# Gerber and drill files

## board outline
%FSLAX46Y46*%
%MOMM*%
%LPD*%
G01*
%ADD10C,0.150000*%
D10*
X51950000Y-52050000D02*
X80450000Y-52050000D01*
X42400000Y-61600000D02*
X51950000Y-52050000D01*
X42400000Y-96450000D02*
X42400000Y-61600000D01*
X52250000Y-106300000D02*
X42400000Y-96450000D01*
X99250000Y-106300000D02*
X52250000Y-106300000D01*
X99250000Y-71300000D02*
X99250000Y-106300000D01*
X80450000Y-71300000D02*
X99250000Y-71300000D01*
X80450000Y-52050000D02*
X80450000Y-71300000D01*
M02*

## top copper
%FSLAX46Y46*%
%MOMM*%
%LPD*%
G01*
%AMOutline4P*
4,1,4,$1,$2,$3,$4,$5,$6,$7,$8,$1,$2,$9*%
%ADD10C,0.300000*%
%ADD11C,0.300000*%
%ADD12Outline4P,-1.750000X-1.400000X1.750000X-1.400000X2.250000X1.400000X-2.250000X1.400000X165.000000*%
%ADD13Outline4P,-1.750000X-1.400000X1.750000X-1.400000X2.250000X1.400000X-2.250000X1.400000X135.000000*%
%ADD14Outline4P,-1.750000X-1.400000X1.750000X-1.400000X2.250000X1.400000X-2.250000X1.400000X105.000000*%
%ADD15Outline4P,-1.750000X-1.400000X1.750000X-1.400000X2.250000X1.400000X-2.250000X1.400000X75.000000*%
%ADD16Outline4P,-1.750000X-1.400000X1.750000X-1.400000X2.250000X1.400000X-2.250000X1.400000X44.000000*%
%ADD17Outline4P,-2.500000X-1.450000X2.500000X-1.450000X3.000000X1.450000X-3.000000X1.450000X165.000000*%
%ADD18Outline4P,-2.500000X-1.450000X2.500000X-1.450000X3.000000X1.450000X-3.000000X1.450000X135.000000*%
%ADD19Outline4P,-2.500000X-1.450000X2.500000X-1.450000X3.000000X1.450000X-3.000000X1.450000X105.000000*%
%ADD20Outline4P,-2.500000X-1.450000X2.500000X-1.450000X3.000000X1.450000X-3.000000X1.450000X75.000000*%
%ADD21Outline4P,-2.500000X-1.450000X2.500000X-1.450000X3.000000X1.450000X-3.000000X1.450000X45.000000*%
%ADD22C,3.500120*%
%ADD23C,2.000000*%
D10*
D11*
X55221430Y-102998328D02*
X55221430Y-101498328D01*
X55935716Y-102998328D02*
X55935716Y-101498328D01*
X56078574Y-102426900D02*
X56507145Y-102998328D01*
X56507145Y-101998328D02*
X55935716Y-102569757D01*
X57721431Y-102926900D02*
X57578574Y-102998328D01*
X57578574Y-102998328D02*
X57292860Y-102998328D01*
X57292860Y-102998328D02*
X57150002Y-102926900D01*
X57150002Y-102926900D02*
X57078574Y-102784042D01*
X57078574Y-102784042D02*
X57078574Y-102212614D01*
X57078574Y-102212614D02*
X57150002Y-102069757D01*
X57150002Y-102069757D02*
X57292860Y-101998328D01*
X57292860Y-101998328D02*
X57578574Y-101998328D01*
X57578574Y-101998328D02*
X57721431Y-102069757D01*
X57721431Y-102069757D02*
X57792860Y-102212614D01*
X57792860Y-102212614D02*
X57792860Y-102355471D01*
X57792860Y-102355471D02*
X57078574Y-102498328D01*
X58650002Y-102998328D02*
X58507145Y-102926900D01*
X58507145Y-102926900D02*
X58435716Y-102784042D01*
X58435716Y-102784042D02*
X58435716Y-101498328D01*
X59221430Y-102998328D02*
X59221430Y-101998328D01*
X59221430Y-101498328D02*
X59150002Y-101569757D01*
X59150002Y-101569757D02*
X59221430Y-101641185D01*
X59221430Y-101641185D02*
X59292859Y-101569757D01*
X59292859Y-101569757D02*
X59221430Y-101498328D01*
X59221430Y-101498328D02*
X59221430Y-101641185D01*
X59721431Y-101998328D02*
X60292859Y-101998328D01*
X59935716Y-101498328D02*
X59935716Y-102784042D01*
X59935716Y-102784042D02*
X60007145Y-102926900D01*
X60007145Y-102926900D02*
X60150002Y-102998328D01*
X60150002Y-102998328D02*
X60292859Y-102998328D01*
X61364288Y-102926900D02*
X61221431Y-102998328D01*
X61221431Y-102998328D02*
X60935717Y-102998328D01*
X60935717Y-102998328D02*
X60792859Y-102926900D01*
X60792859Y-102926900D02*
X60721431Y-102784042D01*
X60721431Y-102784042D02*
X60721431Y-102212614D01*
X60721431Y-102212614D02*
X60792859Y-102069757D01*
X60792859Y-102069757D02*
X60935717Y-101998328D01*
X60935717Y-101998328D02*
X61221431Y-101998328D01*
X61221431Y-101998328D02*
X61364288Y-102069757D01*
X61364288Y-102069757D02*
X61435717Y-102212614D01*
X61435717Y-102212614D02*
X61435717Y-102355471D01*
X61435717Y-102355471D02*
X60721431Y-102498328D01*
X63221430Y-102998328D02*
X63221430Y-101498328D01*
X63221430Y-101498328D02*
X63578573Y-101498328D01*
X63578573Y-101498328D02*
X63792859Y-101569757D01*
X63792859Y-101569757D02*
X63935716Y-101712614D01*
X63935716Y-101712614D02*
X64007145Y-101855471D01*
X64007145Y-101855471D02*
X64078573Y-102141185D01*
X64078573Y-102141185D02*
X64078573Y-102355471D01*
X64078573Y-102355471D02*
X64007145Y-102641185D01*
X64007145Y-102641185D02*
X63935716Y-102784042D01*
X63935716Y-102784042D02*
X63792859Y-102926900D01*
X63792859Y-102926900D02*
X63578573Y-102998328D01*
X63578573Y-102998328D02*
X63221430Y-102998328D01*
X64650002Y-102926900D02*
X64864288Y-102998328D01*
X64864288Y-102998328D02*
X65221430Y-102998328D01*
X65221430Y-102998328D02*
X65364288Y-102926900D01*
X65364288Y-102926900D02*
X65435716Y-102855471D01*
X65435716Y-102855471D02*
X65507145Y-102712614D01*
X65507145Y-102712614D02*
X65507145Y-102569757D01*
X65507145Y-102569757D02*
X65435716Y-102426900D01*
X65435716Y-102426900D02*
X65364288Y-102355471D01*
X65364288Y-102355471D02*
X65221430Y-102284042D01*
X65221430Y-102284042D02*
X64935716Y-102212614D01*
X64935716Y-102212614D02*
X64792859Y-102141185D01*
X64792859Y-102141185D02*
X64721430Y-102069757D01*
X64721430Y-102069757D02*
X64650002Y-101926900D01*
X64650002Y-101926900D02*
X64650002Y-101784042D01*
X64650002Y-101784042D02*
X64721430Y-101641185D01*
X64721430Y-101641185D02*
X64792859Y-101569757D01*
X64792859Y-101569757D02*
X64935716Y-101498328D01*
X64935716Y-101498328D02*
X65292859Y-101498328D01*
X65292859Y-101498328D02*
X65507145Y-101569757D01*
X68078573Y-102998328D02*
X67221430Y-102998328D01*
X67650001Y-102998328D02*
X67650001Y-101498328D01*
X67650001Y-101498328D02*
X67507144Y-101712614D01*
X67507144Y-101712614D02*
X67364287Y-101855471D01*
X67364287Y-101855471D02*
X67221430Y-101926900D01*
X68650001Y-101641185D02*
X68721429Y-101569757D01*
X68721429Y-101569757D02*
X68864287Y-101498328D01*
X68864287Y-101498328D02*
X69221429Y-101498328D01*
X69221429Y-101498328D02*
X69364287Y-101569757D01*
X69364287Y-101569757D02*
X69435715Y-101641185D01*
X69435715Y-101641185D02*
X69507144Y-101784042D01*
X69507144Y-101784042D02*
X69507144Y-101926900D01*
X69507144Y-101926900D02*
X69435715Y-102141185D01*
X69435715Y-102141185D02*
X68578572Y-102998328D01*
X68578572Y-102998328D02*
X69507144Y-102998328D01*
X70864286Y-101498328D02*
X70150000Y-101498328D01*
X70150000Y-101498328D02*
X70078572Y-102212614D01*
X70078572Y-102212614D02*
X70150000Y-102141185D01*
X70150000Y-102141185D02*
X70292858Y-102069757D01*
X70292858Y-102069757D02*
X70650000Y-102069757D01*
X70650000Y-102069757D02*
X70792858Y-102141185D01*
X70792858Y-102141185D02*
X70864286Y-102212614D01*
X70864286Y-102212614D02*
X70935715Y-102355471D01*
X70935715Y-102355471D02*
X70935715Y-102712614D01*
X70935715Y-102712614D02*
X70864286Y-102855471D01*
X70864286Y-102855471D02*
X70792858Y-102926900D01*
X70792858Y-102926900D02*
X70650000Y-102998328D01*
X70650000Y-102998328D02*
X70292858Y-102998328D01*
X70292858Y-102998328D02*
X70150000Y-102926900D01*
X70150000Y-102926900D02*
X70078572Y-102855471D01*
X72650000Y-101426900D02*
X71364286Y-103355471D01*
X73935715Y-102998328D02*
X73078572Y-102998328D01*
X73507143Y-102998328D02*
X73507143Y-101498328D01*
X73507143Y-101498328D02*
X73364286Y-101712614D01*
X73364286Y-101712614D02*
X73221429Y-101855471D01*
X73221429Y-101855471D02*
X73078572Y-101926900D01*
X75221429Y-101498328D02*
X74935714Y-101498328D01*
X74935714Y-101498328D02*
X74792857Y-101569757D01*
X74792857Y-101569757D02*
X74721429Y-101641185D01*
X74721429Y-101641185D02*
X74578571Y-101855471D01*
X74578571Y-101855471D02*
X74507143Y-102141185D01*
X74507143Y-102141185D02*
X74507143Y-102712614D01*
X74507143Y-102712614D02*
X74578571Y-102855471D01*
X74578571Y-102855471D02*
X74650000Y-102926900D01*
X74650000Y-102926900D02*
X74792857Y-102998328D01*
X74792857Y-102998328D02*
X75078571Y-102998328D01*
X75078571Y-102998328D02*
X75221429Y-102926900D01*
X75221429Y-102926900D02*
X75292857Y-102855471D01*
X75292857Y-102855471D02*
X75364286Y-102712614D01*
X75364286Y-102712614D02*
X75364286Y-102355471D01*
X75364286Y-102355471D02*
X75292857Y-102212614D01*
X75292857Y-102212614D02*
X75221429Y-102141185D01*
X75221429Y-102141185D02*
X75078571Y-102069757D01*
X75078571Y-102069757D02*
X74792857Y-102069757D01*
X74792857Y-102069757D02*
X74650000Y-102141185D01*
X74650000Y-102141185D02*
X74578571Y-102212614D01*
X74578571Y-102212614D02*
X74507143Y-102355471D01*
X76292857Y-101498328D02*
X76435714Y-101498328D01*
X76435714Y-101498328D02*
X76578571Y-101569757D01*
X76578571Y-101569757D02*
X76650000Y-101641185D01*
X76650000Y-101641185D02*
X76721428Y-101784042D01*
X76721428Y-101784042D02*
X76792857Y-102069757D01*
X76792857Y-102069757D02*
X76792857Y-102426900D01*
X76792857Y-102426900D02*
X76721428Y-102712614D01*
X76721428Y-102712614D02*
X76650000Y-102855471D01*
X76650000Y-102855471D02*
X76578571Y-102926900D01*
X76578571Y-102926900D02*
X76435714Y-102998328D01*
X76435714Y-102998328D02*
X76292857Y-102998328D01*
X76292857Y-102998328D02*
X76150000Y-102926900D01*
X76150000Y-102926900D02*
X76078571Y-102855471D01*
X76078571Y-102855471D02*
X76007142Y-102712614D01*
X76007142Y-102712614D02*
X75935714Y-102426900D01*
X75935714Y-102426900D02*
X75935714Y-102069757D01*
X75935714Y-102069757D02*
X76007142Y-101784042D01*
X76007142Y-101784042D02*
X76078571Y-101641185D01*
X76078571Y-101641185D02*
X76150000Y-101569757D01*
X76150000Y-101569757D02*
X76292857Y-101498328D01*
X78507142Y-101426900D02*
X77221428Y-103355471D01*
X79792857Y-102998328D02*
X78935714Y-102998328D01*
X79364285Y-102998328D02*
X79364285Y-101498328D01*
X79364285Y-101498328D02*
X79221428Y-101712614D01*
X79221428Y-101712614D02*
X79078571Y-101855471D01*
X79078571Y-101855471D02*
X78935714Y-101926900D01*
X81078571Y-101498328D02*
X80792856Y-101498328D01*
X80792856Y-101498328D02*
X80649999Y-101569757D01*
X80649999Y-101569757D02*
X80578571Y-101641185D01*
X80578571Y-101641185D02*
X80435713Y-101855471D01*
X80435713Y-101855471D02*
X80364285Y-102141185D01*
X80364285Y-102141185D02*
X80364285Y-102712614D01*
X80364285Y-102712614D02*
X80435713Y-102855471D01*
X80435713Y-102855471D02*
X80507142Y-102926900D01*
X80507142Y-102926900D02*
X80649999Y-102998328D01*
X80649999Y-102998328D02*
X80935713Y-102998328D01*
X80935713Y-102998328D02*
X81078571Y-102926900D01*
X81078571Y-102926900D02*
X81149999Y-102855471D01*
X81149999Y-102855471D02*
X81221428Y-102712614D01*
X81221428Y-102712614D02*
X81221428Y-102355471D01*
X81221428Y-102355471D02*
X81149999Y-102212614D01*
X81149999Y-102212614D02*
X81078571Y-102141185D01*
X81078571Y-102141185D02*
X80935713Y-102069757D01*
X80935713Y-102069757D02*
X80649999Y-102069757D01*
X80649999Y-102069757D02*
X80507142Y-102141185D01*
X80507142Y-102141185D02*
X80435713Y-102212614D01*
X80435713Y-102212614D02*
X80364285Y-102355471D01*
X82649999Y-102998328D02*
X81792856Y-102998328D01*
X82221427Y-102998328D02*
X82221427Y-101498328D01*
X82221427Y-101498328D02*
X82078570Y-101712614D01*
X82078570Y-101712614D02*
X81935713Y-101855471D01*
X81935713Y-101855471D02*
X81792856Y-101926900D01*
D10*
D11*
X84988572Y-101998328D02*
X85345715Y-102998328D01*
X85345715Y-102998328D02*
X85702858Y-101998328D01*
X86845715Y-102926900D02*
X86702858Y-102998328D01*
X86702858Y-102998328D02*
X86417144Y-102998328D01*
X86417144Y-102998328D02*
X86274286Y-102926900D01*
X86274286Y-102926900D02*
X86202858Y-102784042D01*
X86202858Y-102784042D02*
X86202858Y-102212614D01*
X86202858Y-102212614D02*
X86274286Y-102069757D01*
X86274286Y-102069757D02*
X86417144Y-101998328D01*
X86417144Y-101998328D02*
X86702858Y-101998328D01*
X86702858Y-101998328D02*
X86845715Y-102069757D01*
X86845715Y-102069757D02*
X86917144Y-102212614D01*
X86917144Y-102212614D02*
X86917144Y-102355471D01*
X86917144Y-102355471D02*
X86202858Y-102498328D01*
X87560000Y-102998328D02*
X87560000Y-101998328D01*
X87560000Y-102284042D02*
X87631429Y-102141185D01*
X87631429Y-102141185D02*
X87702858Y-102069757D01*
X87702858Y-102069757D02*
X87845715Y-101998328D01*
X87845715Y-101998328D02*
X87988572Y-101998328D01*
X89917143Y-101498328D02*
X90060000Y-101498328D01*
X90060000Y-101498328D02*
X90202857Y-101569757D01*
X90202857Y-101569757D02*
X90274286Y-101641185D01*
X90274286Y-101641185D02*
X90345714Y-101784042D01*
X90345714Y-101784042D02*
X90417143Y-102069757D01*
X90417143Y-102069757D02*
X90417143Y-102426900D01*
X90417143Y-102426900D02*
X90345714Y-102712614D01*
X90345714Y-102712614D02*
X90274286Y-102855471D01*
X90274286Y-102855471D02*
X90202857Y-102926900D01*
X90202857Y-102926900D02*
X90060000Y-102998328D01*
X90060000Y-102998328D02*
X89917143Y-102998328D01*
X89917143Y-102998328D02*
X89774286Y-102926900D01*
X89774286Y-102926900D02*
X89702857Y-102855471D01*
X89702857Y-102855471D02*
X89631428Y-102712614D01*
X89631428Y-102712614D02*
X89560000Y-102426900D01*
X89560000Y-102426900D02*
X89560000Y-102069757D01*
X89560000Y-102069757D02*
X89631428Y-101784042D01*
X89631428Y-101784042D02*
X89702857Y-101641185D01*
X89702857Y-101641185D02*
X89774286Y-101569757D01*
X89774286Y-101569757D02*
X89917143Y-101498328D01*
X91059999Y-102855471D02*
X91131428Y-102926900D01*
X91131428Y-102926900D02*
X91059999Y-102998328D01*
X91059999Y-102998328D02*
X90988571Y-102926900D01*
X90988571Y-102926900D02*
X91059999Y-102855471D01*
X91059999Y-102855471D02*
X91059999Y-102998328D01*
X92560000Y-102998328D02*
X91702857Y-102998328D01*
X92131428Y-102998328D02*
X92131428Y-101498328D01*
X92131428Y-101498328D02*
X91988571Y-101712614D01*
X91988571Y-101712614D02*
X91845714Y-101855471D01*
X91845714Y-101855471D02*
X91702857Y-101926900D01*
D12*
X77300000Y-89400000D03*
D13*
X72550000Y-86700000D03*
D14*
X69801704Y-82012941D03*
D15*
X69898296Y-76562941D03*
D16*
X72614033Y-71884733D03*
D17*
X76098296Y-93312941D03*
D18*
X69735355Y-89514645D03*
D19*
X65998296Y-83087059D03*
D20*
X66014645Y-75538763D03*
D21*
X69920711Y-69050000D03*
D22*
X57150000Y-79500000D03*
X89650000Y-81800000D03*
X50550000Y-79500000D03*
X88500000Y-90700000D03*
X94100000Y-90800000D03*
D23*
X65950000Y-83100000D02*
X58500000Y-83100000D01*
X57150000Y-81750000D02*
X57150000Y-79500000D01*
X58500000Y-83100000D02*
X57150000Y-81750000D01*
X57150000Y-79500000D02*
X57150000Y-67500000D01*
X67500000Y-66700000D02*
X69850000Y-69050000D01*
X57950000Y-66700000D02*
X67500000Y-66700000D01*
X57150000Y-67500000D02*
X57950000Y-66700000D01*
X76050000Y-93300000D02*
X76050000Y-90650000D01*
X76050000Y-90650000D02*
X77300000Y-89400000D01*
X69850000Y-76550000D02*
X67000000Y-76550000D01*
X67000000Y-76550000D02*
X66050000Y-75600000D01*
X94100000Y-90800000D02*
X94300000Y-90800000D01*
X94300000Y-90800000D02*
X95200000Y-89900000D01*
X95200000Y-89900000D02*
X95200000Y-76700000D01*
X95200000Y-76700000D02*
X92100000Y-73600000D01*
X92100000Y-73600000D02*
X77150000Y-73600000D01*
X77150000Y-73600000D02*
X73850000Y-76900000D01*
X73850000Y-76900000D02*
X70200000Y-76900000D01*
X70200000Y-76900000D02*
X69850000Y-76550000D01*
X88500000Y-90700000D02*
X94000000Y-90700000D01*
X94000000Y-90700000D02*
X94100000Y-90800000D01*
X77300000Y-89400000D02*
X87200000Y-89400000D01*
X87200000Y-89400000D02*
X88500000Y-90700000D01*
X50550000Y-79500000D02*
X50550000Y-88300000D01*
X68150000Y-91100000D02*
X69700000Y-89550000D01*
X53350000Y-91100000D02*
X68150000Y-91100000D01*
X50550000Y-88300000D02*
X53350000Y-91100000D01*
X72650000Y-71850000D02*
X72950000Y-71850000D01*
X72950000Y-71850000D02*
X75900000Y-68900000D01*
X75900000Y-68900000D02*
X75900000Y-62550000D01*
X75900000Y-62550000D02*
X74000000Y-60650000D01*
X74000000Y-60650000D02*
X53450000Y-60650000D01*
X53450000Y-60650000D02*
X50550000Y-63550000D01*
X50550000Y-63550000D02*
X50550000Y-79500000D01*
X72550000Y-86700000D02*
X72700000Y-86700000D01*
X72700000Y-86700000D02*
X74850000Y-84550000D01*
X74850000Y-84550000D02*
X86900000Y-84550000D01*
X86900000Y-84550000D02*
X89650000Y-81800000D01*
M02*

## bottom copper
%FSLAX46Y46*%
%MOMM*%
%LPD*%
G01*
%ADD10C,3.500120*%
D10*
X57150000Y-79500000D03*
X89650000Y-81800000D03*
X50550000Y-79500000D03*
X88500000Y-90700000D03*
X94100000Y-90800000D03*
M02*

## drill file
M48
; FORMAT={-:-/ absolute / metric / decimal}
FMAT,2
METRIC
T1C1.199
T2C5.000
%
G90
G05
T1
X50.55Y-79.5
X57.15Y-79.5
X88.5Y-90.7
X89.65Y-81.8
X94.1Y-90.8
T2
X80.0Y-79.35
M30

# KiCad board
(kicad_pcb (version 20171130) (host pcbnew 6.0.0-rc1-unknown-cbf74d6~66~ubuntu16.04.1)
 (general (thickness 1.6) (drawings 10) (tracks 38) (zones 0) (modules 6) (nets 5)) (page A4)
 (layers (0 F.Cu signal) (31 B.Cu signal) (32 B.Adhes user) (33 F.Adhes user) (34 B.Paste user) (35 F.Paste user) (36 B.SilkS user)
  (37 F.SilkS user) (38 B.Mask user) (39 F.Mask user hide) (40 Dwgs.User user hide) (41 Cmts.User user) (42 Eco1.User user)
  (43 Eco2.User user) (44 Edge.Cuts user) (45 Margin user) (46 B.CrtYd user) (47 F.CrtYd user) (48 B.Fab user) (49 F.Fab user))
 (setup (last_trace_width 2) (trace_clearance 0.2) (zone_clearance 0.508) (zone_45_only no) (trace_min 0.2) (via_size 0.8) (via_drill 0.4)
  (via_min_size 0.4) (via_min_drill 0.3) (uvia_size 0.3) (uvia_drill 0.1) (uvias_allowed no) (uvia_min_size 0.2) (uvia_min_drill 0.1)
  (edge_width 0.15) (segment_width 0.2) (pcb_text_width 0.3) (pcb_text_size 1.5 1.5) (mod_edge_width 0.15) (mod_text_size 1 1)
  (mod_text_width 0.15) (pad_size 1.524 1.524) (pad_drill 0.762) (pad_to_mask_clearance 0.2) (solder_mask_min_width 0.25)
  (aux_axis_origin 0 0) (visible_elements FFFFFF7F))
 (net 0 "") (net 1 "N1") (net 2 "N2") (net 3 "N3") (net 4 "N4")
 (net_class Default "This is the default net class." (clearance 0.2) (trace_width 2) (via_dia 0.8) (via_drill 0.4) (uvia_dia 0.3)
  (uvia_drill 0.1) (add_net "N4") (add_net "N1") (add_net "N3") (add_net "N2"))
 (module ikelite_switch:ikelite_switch (layer F.Cu) (at 80 79.4)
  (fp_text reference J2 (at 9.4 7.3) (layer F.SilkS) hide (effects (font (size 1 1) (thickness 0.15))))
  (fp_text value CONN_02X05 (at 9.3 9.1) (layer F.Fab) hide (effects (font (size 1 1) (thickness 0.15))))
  (pad 10 connect trapezoid (at -2.7 10 165) (size 4 2.8) (rect_delta 0 -0.5) (layers F.Cu F.Mask) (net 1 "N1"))
  (pad 8 connect trapezoid (at -7.45 7.3 135) (size 4 2.8) (rect_delta 0 -0.5) (layers F.Cu F.Mask) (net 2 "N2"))
  (pad 6 connect trapezoid (at -10.15 2.6 105) (size 4 2.8) (rect_delta 0 -0.5) (drill (offset 0 -0.05)) (layers F.Cu F.Mask))
  (pad 4 connect trapezoid (at -10.15 -2.85 75) (size 4 2.8) (rect_delta 0 -0.5) (drill (offset 0 0.05)) (layers F.Cu F.Mask) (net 1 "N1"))
  (pad 2 connect trapezoid (at -7.35 -7.55 44) (size 4 2.8) (rect_delta 0 -0.5) (drill (offset -0.05 0)) (layers F.Cu F.Mask) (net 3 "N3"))
  (pad 9 connect trapezoid (at -3.95 13.9 165) (size 5.5 2.9) (rect_delta 0 -0.5) (drill (offset -0.05 0)) (layers F.Cu F.Mask) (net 1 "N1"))
  (pad 7 connect trapezoid (at -10.3 10.15 135) (size 5.5 2.9) (rect_delta 0 -0.5) (drill (offset 0 0.05)) (layers F.Cu F.Mask) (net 3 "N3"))
  (pad 5 connect trapezoid (at -14.05 3.7 105) (size 5.5 2.9) (rect_delta 0 -0.5) (drill (offset 0 0.05)) (layers F.Cu F.Mask) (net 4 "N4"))
  (pad 3 connect trapezoid (at -13.95 -3.8 75) (size 5.5 2.9) (rect_delta 0 -0.5) (drill (offset 0.05 -0.05)) (layers F.Cu F.Mask)
   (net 1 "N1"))
  (pad 1 connect trapezoid (at -10.15 -10.35 45) (size 5.5 2.9) (rect_delta 0 -0.5) (drill (offset 0.05 0.05)) (layers F.Cu F.Mask)
   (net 4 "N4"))
  (pad "" np_thru_hole circle (at 0 -0.05) (size 5 5) (drill 5) (layers *.Cu *.Mask)))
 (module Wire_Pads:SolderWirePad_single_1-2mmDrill (layer F.Cu) (at 57.15 79.5)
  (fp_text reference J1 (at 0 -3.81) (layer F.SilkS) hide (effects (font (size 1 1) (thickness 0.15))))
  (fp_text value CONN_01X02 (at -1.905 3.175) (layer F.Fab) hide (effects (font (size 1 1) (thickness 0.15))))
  (pad 1 thru_hole circle (at 0 0) (size 3.50012 3.50012) (drill 1.19888) (layers *.Cu *.Mask) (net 4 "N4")))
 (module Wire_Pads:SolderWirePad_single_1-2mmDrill (layer F.Cu) (at 89.65 81.8)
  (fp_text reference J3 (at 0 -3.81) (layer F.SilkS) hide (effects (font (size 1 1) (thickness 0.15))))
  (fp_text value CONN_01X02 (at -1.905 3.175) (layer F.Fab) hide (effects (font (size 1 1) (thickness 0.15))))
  (pad 1 thru_hole circle (at 0 0) (size 3.50012 3.50012) (drill 1.19888) (layers *.Cu *.Mask) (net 2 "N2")))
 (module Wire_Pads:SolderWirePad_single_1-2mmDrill (layer F.Cu) (at 50.55 79.5)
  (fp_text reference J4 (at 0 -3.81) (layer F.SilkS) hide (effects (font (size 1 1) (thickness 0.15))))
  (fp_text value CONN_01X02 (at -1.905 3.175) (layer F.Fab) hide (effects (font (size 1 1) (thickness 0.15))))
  (pad 1 thru_hole circle (at 0 0) (size 3.50012 3.50012) (drill 1.19888) (layers *.Cu *.Mask) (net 3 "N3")))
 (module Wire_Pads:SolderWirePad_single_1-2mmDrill (layer F.Cu) (at 88.5 90.7)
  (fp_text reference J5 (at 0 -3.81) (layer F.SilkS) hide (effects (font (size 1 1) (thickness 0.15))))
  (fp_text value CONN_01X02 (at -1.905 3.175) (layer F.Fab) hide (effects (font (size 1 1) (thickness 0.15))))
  (pad 1 thru_hole circle (at 0 0) (size 3.50012 3.50012) (drill 1.19888) (layers *.Cu *.Mask) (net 1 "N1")))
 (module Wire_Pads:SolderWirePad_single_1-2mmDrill (layer F.Cu) (at 94.1 90.8)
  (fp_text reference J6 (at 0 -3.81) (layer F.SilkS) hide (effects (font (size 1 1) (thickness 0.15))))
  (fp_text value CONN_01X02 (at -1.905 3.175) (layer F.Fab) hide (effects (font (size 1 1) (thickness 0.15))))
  (pad 1 thru_hole circle (at 0 0) (size 3.50012 3.50012) (drill 1.19888) (layers *.Cu *.Mask) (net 1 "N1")))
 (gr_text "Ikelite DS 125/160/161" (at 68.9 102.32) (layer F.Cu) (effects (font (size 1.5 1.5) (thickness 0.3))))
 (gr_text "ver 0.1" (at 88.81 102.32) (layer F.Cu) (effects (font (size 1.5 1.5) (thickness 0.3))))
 (gr_line (start 51.95 52.05) (end 80.45 52.05) (angle 90) (layer Edge.Cuts) (width 0.15))
 (gr_line (start 42.4 61.6) (end 51.95 52.05) (angle 90) (layer Edge.Cuts) (width 0.15))
 (gr_line (start 42.4 96.45) (end 42.4 61.6) (angle 90) (layer Edge.Cuts) (width 0.15))
 (gr_line (start 52.25 106.3) (end 42.4 96.45) (angle 90) (layer Edge.Cuts) (width 0.15))
 (gr_line (start 99.25 106.3) (end 52.25 106.3) (angle 90) (layer Edge.Cuts) (width 0.15))
 (gr_line (start 99.25 71.3) (end 99.25 106.3) (angle 90) (layer Edge.Cuts) (width 0.15))
 (gr_line (start 80.45 71.3) (end 99.25 71.3) (angle 90) (layer Edge.Cuts) (width 0.15))
 (gr_line (start 80.45 52.05) (end 80.45 71.3) (angle 90) (layer Edge.Cuts) (width 0.15))
 (segment (start 65.95 83.1) (end 58.5 83.1) (width 2) (layer F.Cu) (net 4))
 (segment (start 57.15 81.75) (end 57.15 79.5) (width 2) (layer F.Cu) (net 4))
 (segment (start 58.5 83.1) (end 57.15 81.75) (width 2) (layer F.Cu) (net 4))
 (segment (start 57.15 79.5) (end 57.15 67.5) (width 2) (layer F.Cu) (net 4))
 (segment (start 67.5 66.7) (end 69.85 69.05) (width 2) (layer F.Cu) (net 4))
 (segment (start 57.95 66.7) (end 67.5 66.7) (width 2) (layer F.Cu) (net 4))
 (segment (start 57.15 67.5) (end 57.95 66.7) (width 2) (layer F.Cu) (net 4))
 (segment (start 76.05 93.3) (end 76.05 90.65) (width 2) (layer F.Cu) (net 1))
 (segment (start 76.05 90.65) (end 77.3 89.4) (width 2) (layer F.Cu) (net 1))
 (segment (start 69.85 76.55) (end 67 76.55) (width 2) (layer F.Cu) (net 1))
 (segment (start 67 76.55) (end 66.05 75.6) (width 2) (layer F.Cu) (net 1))
 (segment (start 94.1 90.8) (end 94.3 90.8) (width 2) (layer F.Cu) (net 1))
 (segment (start 94.3 90.8) (end 95.2 89.9) (width 2) (layer F.Cu) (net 1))
 (segment (start 95.2 89.9) (end 95.2 76.7) (width 2) (layer F.Cu) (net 1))
 (segment (start 95.2 76.7) (end 92.1 73.6) (width 2) (layer F.Cu) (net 1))
 (segment (start 92.1 73.6) (end 77.15 73.6) (width 2) (layer F.Cu) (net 1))
 (segment (start 77.15 73.6) (end 73.85 76.9) (width 2) (layer F.Cu) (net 1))
 (segment (start 73.85 76.9) (end 70.2 76.9) (width 2) (layer F.Cu) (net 1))
 (segment (start 70.2 76.9) (end 69.85 76.55) (width 2) (layer F.Cu) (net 1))
 (segment (start 88.5 90.7) (end 94 90.7) (width 2) (layer F.Cu) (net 1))
 (segment (start 94 90.7) (end 94.1 90.8) (width 2) (layer F.Cu) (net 1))
 (segment (start 77.3 89.4) (end 87.2 89.4) (width 2) (layer F.Cu) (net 1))
 (segment (start 87.2 89.4) (end 88.5 90.7) (width 2) (layer F.Cu) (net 1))
 (segment (start 50.55 79.5) (end 50.55 88.3) (width 2) (layer F.Cu) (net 3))
 (segment (start 68.15 91.1) (end 69.7 89.55) (width 2) (layer F.Cu) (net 3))
 (segment (start 53.35 91.1) (end 68.15 91.1) (width 2) (layer F.Cu) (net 3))
 (segment (start 50.55 88.3) (end 53.35 91.1) (width 2) (layer F.Cu) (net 3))
 (segment (start 72.65 71.85) (end 72.95 71.85) (width 2) (layer F.Cu) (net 3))
 (segment (start 72.95 71.85) (end 75.9 68.9) (width 2) (layer F.Cu) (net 3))
 (segment (start 75.9 68.9) (end 75.9 62.55) (width 2) (layer F.Cu) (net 3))
 (segment (start 75.9 62.55) (end 74 60.65) (width 2) (layer F.Cu) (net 3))
 (segment (start 74 60.65) (end 53.45 60.65) (width 2) (layer F.Cu) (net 3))
 (segment (start 53.45 60.65) (end 50.55 63.55) (width 2) (layer F.Cu) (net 3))
 (segment (start 50.55 63.55) (end 50.55 79.5) (width 2) (layer F.Cu) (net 3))
 (segment (start 72.55 86.7) (end 72.7 86.7) (width 2) (layer F.Cu) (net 2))
 (segment (start 72.7 86.7) (end 74.85 84.55) (width 2) (layer F.Cu) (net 2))
 (segment (start 74.85 84.55) (end 86.9 84.55) (width 2) (layer F.Cu) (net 2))
 (segment (start 86.9 84.55) (end 89.65 81.8) (width 2) (layer F.Cu) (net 2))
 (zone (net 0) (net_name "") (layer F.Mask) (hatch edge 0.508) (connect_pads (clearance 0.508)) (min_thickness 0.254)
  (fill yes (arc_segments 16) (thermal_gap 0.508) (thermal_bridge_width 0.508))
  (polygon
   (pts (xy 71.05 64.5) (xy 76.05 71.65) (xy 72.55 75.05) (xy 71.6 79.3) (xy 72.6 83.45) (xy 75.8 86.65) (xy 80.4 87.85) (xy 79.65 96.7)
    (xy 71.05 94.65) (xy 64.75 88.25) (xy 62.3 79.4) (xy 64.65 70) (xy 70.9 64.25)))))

